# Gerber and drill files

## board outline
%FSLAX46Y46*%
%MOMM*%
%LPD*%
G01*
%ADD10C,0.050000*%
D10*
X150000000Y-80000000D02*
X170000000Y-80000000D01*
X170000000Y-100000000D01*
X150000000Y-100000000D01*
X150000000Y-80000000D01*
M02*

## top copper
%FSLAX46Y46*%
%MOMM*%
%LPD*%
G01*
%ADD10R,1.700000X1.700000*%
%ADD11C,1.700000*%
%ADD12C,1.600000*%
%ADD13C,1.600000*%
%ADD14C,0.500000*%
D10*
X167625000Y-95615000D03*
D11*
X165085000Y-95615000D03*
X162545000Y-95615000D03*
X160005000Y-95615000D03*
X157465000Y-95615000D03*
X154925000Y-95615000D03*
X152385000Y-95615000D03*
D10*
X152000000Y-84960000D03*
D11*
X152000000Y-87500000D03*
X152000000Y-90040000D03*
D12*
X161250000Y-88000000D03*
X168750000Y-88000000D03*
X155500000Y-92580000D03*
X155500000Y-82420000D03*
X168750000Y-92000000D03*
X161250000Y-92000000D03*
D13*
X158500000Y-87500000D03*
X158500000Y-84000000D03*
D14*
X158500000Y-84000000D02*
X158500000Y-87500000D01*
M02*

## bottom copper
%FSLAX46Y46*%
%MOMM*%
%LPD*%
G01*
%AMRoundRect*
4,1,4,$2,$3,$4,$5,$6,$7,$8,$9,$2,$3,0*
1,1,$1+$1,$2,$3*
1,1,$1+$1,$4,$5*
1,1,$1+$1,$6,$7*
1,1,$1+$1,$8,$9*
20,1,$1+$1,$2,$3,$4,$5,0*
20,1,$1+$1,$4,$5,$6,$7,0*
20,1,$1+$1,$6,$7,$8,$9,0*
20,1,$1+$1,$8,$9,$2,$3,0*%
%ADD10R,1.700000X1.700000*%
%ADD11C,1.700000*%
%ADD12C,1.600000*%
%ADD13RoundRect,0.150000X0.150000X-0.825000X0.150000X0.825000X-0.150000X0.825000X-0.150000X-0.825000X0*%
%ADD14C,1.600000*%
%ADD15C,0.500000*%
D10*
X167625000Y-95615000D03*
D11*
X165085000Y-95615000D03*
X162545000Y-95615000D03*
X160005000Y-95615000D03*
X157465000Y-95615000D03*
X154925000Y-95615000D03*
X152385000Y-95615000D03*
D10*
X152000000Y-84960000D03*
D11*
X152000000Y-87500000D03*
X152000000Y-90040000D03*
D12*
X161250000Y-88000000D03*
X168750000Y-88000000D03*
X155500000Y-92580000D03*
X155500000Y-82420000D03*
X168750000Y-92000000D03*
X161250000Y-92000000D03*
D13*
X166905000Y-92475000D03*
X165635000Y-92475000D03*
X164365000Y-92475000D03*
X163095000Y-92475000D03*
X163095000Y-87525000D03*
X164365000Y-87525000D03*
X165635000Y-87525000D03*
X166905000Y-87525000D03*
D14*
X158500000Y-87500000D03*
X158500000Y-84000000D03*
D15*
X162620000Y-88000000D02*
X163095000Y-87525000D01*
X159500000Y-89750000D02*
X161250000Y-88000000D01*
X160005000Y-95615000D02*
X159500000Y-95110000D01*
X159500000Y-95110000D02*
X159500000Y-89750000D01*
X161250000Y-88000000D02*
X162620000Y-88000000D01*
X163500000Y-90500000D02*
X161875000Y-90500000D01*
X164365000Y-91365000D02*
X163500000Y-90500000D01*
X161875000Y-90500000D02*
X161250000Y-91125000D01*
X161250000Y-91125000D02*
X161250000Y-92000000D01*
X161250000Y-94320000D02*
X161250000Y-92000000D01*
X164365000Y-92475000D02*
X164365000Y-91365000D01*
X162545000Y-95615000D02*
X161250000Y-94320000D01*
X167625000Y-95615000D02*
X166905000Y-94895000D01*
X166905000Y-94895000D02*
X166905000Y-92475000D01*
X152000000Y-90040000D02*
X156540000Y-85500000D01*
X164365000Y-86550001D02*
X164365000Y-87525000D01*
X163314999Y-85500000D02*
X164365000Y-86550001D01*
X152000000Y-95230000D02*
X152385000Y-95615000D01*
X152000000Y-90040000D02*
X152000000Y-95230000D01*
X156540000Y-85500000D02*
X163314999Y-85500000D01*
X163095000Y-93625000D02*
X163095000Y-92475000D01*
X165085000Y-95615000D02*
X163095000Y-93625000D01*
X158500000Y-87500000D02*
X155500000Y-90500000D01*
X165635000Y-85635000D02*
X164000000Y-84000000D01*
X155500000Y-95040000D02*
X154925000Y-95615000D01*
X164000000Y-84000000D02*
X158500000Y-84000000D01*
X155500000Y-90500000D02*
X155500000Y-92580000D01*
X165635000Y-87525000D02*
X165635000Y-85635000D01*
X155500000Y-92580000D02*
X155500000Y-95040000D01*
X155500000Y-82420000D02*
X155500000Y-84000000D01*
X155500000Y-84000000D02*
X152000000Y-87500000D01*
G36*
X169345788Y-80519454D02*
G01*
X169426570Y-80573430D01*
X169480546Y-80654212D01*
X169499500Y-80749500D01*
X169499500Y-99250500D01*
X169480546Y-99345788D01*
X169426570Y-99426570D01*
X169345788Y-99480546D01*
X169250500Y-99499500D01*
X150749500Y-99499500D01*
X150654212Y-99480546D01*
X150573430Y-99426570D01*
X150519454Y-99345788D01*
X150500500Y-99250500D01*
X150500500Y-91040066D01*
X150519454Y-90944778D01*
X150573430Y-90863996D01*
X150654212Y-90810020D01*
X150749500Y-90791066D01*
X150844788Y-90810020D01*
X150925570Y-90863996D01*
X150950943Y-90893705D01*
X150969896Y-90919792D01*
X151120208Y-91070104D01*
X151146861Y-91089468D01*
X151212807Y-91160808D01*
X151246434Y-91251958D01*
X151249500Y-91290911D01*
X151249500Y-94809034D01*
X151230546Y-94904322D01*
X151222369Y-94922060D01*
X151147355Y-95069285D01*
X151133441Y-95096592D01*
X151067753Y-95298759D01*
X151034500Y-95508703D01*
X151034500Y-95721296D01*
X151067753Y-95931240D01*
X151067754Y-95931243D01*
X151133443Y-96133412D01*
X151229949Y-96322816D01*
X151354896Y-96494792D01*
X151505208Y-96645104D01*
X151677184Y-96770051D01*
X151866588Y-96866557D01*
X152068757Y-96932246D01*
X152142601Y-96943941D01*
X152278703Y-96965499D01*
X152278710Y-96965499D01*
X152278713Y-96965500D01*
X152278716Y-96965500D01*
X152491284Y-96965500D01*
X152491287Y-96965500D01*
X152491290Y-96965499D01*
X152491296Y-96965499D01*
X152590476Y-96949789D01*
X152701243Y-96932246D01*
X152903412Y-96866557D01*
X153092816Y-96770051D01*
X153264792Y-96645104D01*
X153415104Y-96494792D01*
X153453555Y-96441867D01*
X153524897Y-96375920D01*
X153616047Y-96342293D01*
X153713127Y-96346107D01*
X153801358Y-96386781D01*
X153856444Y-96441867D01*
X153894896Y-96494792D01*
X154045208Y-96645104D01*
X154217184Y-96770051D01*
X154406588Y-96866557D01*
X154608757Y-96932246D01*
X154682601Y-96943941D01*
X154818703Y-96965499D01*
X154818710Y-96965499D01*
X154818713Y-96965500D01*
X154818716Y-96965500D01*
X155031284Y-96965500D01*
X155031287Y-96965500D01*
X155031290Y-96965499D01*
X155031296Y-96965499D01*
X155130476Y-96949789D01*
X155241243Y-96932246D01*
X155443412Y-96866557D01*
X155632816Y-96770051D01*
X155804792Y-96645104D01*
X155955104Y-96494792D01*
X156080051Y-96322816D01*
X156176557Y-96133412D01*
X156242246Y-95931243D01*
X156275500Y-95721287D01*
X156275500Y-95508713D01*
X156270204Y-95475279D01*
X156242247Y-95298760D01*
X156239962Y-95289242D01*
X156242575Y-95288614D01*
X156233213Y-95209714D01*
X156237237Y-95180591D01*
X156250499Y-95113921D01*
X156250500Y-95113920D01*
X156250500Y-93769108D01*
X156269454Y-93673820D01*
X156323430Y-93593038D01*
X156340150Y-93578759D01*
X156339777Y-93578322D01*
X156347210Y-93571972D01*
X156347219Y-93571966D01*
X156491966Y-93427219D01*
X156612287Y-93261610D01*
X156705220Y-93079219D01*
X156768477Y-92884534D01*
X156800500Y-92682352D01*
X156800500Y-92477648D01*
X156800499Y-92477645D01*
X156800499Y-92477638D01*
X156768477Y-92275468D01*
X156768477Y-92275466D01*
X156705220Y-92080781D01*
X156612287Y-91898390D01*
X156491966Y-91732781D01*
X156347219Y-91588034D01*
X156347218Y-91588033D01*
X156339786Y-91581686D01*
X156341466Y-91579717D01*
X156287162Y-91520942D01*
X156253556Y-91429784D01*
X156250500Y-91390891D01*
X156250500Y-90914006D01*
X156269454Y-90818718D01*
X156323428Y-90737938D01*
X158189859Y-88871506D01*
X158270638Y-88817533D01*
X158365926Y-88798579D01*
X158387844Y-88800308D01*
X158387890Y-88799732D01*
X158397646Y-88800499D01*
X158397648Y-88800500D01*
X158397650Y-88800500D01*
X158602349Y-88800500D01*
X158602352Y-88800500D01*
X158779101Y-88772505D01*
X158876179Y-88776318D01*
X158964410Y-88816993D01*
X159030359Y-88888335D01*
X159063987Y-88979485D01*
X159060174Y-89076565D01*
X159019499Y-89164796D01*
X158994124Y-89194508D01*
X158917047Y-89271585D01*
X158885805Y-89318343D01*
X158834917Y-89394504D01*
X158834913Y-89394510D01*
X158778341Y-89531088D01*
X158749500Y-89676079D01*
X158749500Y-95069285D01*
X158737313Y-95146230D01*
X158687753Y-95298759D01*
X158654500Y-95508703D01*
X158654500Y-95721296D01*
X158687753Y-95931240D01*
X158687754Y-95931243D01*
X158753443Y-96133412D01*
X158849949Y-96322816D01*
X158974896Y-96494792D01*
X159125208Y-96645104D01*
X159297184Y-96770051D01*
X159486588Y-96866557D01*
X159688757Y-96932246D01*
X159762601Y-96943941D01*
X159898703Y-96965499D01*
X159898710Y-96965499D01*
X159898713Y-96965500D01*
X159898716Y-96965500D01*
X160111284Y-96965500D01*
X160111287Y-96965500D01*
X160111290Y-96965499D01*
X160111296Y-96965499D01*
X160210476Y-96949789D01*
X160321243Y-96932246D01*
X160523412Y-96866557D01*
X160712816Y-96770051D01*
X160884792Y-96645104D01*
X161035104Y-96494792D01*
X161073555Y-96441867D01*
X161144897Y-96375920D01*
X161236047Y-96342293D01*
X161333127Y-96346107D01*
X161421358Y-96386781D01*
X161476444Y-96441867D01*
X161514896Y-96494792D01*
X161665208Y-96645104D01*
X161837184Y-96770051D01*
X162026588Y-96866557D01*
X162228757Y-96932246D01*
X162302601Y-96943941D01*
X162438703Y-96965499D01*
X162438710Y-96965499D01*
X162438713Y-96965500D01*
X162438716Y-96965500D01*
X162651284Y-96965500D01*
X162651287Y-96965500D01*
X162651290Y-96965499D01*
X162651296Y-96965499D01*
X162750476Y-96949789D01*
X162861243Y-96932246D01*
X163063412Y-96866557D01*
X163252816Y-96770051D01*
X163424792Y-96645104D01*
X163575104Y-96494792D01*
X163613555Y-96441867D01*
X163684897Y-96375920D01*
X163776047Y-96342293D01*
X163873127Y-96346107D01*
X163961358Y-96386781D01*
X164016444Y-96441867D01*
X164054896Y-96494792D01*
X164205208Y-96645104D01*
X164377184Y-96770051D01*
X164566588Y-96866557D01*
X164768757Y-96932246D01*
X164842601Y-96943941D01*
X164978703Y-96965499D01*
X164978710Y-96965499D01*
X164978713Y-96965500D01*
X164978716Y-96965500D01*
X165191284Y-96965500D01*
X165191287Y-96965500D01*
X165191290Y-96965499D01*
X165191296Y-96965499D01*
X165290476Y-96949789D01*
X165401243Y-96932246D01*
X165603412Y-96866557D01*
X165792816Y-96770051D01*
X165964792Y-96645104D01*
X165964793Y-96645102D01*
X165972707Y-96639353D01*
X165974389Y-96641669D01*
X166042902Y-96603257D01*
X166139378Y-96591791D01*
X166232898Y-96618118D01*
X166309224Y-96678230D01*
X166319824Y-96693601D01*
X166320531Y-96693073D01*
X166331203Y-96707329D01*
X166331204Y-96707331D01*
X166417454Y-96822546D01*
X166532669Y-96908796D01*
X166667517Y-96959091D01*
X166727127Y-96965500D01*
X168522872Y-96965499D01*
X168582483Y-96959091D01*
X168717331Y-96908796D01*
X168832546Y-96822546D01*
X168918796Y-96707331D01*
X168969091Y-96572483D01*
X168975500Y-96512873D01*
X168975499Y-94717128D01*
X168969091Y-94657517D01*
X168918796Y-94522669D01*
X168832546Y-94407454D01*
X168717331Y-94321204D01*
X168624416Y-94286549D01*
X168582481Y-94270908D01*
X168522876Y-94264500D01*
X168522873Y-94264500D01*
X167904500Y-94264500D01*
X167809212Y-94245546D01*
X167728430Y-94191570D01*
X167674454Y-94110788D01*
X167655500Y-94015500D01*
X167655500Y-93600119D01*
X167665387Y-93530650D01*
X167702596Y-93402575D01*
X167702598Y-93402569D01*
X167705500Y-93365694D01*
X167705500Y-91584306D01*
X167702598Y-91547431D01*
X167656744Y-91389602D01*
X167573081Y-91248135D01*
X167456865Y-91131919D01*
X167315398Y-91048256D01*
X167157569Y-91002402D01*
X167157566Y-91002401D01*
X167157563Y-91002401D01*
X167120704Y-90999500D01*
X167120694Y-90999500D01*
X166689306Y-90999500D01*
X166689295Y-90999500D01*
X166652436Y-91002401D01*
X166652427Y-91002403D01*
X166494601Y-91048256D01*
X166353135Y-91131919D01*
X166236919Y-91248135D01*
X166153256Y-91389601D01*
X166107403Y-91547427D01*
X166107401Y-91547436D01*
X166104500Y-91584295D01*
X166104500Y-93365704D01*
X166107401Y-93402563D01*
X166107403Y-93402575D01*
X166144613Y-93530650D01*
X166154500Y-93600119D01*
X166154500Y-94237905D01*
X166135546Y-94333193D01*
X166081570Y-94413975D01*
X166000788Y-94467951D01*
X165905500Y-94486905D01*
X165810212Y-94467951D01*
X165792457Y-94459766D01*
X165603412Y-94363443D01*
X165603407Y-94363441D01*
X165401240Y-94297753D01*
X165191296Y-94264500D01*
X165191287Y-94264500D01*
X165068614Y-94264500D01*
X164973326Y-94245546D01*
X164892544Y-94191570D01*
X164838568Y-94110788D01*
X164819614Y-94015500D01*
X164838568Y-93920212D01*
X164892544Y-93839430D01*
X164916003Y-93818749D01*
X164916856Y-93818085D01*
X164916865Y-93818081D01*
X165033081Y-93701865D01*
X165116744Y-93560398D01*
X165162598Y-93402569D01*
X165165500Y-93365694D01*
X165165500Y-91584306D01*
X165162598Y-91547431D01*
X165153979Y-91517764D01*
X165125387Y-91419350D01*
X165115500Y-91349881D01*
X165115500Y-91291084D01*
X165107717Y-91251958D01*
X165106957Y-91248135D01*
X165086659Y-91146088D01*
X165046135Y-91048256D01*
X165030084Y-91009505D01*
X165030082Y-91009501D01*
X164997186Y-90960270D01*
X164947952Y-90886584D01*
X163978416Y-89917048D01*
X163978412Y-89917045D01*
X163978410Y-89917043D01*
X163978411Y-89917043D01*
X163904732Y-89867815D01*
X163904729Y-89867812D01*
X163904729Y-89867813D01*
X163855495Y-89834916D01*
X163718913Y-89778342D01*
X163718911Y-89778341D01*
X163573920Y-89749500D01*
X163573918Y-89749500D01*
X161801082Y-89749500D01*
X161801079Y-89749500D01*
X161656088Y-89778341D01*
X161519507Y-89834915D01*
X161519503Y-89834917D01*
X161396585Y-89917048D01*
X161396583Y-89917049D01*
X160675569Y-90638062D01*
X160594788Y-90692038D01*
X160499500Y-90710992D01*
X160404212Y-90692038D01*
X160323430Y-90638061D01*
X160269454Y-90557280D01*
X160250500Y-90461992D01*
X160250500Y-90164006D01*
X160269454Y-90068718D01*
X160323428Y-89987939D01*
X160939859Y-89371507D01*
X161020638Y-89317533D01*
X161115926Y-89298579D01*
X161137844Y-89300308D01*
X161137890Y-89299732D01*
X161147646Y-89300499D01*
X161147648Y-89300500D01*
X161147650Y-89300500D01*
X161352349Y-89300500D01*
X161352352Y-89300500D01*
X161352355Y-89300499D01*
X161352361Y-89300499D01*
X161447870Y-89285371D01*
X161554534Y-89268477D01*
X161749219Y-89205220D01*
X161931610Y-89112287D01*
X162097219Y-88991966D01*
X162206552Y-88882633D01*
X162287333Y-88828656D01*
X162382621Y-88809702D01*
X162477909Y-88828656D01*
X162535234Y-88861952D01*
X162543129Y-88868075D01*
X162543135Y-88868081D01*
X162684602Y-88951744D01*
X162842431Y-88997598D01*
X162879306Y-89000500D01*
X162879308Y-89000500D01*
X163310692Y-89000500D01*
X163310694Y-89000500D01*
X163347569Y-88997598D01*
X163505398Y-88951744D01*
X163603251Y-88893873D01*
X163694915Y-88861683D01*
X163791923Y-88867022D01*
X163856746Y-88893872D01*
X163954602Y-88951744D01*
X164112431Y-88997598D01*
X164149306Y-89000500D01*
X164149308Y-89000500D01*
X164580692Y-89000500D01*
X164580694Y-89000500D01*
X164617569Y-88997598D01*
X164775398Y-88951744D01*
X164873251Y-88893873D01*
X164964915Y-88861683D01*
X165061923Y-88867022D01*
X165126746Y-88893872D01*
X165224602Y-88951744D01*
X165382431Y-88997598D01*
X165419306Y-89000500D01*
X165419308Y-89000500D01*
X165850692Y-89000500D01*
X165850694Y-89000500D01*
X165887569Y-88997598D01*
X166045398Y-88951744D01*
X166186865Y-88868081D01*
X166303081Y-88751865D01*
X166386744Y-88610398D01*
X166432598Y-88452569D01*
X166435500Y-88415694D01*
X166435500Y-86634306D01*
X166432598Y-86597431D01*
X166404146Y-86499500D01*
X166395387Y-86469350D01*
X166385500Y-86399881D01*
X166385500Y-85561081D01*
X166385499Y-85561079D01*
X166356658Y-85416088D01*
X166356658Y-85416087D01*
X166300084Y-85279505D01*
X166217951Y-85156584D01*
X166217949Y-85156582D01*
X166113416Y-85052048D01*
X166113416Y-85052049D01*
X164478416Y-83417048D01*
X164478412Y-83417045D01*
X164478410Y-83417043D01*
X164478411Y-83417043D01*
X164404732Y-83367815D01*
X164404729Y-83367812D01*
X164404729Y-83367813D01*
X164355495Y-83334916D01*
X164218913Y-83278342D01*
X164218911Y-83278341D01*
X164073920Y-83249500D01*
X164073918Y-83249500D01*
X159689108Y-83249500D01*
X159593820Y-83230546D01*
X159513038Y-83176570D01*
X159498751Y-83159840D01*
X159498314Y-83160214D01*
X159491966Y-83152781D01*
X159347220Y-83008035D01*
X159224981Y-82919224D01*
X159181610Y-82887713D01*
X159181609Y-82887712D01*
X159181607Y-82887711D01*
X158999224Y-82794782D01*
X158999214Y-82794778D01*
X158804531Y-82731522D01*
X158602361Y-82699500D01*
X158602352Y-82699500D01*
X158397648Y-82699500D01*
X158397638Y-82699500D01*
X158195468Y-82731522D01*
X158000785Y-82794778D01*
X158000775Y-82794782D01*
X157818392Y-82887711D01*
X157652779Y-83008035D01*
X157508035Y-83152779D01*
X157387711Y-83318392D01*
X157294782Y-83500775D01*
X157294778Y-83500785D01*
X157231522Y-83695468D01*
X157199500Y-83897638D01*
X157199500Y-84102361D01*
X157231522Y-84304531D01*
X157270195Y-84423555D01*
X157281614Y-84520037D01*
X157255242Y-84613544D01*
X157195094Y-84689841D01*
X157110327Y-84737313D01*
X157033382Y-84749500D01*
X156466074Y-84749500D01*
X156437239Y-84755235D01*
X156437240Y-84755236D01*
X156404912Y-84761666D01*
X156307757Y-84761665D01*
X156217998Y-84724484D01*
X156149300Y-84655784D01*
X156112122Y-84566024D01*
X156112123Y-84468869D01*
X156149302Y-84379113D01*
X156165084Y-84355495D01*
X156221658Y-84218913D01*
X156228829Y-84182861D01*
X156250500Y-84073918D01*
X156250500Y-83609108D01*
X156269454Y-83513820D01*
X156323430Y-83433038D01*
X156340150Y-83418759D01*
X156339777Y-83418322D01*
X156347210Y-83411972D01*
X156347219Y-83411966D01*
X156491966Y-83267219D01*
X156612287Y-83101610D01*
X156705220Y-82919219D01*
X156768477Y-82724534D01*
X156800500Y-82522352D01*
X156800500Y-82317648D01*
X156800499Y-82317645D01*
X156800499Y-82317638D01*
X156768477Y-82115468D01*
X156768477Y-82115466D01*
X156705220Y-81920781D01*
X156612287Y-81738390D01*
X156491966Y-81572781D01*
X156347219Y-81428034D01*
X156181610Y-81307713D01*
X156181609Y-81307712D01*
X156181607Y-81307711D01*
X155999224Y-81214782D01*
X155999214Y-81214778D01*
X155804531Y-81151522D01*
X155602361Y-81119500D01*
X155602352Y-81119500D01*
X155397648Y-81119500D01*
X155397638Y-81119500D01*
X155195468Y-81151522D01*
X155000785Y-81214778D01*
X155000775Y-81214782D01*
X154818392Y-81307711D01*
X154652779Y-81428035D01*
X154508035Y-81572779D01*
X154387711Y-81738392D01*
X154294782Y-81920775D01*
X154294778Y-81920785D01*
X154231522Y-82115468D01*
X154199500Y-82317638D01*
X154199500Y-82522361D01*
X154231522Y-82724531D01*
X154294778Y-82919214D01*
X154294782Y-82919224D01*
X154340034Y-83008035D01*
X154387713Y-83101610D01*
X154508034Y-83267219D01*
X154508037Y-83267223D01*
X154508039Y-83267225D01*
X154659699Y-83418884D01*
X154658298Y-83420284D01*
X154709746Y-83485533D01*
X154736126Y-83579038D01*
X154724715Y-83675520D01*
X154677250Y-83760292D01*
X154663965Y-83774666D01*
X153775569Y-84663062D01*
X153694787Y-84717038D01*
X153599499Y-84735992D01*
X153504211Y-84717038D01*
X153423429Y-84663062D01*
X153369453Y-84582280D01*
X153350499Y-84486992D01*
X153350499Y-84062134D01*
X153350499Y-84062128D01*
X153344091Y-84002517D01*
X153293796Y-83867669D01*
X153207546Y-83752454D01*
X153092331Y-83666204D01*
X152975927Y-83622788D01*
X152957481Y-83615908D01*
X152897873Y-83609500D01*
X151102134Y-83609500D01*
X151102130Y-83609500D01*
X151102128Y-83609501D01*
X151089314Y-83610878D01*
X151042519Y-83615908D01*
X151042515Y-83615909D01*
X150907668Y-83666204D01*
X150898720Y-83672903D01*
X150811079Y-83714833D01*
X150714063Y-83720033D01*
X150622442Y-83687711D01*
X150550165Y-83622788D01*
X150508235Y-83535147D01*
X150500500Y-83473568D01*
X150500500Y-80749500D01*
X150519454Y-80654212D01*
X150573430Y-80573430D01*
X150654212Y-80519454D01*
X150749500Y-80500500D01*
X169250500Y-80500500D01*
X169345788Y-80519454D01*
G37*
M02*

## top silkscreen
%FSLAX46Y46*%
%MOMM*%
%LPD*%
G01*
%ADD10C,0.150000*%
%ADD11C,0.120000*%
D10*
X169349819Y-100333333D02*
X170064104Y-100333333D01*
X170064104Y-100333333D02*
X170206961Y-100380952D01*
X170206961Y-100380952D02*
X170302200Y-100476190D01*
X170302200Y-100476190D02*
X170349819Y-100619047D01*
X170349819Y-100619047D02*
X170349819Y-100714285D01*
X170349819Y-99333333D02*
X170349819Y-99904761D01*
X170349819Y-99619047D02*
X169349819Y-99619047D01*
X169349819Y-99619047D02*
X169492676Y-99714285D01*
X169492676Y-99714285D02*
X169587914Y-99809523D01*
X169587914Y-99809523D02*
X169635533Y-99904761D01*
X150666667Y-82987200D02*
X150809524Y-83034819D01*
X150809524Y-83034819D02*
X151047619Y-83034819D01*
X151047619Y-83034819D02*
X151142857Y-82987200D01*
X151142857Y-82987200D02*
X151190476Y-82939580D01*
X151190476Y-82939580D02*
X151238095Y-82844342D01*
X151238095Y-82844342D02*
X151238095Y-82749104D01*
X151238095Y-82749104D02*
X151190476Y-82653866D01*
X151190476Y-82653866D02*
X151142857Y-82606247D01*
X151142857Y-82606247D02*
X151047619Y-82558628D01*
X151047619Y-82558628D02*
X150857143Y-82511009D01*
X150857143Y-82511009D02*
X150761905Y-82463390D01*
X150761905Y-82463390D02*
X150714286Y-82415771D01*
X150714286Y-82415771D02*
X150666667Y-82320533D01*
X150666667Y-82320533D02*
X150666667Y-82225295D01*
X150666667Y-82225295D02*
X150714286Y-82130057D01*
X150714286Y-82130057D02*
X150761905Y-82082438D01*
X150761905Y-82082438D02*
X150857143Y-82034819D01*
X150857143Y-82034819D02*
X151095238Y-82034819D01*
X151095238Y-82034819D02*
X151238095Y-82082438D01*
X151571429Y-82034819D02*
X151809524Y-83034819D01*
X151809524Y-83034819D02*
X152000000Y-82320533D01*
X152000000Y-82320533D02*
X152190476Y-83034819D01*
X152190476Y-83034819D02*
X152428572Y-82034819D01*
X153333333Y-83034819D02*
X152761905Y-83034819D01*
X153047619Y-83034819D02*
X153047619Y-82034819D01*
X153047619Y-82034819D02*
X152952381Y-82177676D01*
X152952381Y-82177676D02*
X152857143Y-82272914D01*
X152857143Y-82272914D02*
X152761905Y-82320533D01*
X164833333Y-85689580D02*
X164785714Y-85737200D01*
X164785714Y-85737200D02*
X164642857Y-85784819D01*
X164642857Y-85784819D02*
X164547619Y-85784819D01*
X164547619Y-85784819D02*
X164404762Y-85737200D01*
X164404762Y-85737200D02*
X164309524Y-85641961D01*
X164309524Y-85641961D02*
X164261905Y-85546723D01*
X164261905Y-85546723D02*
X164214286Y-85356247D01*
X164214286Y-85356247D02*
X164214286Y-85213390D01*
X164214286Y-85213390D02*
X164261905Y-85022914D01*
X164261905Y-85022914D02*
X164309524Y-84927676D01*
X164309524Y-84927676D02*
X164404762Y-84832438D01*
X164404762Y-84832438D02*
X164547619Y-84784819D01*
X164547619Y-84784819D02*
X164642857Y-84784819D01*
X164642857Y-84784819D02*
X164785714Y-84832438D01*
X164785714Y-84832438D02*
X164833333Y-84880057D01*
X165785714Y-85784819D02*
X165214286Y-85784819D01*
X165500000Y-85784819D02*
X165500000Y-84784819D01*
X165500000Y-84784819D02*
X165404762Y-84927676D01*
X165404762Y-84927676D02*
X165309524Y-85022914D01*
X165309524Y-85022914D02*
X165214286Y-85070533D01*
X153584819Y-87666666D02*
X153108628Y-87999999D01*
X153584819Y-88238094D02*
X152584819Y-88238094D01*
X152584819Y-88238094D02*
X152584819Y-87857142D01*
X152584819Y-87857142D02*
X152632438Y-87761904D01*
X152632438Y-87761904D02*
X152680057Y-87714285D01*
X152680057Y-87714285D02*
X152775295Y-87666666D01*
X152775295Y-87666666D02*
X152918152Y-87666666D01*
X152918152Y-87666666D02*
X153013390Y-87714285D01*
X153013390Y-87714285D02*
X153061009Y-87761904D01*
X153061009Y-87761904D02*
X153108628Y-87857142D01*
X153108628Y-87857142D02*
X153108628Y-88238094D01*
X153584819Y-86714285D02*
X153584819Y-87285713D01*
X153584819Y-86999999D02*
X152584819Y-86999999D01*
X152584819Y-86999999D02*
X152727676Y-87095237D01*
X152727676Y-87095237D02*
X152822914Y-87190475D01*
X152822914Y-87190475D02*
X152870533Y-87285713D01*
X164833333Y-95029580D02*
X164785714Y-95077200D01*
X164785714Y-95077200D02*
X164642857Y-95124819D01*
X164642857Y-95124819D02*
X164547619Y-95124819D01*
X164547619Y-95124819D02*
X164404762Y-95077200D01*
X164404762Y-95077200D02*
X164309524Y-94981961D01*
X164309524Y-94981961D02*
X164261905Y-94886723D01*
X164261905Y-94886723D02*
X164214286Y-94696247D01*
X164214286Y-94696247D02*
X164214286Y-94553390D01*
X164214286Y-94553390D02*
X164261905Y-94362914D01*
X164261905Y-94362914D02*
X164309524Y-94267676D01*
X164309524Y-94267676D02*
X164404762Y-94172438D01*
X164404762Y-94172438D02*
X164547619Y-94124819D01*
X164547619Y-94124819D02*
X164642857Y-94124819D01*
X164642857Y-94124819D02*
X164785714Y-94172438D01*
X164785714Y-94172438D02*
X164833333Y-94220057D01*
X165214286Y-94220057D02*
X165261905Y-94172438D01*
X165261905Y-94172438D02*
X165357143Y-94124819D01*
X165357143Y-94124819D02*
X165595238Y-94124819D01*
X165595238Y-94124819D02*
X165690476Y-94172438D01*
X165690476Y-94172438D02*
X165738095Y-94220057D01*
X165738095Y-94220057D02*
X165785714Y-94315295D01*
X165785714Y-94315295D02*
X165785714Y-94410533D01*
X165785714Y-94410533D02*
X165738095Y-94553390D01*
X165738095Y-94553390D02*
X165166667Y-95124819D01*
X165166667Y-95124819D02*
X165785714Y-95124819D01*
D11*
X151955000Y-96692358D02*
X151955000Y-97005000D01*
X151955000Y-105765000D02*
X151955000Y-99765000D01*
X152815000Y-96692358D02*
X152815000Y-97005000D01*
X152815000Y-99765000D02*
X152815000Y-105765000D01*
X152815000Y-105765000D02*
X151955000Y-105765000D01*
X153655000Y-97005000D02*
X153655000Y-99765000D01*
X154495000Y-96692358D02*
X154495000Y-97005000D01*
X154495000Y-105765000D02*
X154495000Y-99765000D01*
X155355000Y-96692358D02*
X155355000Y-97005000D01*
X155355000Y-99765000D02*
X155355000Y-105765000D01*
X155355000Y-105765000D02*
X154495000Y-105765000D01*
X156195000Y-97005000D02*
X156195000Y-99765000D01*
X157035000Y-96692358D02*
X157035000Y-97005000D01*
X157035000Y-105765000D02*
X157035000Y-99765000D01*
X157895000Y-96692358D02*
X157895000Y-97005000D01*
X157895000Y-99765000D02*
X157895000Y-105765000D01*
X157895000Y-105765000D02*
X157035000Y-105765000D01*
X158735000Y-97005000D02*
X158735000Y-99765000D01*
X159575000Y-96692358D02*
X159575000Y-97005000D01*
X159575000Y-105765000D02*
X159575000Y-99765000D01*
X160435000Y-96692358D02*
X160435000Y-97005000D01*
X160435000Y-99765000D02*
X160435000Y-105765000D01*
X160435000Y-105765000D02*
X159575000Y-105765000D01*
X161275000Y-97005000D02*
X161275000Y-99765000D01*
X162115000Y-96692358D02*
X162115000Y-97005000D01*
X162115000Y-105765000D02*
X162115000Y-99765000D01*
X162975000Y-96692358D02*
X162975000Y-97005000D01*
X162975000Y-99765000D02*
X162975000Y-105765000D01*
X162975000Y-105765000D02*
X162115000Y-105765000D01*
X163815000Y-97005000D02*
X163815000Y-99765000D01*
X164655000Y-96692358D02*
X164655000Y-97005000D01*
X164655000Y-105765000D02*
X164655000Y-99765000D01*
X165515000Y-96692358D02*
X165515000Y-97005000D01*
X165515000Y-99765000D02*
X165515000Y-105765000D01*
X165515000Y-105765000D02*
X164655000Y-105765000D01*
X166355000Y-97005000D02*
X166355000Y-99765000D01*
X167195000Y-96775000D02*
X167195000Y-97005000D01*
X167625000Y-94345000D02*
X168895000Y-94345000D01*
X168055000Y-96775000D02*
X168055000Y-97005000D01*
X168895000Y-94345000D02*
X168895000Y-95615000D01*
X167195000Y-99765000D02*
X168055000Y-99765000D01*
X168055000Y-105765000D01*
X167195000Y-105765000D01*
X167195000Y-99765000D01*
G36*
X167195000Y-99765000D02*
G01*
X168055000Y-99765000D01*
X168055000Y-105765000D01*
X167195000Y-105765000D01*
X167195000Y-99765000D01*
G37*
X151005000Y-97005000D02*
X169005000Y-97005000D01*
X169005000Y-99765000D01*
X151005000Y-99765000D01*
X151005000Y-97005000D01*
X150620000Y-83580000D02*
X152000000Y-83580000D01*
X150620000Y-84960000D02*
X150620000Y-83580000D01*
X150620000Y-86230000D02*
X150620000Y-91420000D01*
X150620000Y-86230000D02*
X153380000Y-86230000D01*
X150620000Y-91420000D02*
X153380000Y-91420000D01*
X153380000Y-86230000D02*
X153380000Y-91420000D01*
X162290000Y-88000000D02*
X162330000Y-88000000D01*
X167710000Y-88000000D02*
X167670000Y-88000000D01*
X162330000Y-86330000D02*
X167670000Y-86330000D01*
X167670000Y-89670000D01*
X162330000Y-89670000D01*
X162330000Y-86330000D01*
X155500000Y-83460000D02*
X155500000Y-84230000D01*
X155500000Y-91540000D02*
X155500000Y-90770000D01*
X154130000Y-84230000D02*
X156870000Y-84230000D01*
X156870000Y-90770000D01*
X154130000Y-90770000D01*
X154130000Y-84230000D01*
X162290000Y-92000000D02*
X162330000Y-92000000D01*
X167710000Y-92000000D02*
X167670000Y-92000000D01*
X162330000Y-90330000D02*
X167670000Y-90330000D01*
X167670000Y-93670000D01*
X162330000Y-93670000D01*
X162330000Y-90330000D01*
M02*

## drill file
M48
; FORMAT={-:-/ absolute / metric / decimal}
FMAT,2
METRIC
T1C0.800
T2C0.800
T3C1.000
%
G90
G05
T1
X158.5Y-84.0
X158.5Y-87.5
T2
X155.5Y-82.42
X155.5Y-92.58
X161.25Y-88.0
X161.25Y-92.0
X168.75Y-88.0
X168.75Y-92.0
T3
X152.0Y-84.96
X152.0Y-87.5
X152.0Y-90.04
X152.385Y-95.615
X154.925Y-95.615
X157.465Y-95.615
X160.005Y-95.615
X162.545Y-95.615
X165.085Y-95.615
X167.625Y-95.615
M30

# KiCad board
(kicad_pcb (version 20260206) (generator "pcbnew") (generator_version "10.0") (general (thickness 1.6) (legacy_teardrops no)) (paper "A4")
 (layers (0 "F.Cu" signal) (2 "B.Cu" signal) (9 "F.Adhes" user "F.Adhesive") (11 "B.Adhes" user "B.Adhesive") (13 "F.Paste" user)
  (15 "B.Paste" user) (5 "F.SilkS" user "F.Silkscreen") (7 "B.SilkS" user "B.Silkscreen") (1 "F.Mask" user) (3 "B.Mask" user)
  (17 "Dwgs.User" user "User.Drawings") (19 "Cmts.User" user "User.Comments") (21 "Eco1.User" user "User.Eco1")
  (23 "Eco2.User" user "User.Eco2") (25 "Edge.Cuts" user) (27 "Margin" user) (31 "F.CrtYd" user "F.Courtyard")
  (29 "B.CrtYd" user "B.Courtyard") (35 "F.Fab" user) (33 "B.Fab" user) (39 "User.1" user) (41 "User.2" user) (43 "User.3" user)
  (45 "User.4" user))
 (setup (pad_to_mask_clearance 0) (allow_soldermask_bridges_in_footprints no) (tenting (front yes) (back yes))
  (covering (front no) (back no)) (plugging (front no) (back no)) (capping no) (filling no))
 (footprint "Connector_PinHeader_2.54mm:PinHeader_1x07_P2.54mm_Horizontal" (layer "F.Cu") (at 167.625 95.615 -90)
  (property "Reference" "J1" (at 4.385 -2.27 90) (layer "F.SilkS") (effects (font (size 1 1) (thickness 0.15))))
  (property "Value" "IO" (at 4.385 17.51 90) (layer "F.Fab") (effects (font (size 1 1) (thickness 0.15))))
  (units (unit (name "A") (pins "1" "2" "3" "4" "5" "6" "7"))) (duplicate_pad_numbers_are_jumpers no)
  (fp_line (start 1.077358 15.67) (end 1.39 15.67) (stroke (width 0.12) (type solid)) (layer "F.SilkS"))
  (fp_line (start 10.15 15.67) (end 4.15 15.67) (stroke (width 0.12) (type solid)) (layer "F.SilkS"))
  (fp_line (start 1.077358 14.81) (end 1.39 14.81) (stroke (width 0.12) (type solid)) (layer "F.SilkS"))
  (fp_line (start 4.15 14.81) (end 10.15 14.81) (stroke (width 0.12) (type solid)) (layer "F.SilkS"))
  (fp_line (start 10.15 14.81) (end 10.15 15.67) (stroke (width 0.12) (type solid)) (layer "F.SilkS"))
  (fp_line (start 1.39 13.97) (end 4.15 13.97) (stroke (width 0.12) (type solid)) (layer "F.SilkS"))
  (fp_line (start 1.077358 13.13) (end 1.39 13.13) (stroke (width 0.12) (type solid)) (layer "F.SilkS"))
  (fp_line (start 10.15 13.13) (end 4.15 13.13) (stroke (width 0.12) (type solid)) (layer "F.SilkS"))
  (fp_line (start 1.077358 12.27) (end 1.39 12.27) (stroke (width 0.12) (type solid)) (layer "F.SilkS"))
  (fp_line (start 4.15 12.27) (end 10.15 12.27) (stroke (width 0.12) (type solid)) (layer "F.SilkS"))
  (fp_line (start 10.15 12.27) (end 10.15 13.13) (stroke (width 0.12) (type solid)) (layer "F.SilkS"))
  (fp_line (start 1.39 11.43) (end 4.15 11.43) (stroke (width 0.12) (type solid)) (layer "F.SilkS"))
  (fp_line (start 1.077358 10.59) (end 1.39 10.59) (stroke (width 0.12) (type solid)) (layer "F.SilkS"))
  (fp_line (start 10.15 10.59) (end 4.15 10.59) (stroke (width 0.12) (type solid)) (layer "F.SilkS"))
  (fp_line (start 1.077358 9.73) (end 1.39 9.73) (stroke (width 0.12) (type solid)) (layer "F.SilkS"))
  (fp_line (start 4.15 9.73) (end 10.15 9.73) (stroke (width 0.12) (type solid)) (layer "F.SilkS"))
  (fp_line (start 10.15 9.73) (end 10.15 10.59) (stroke (width 0.12) (type solid)) (layer "F.SilkS"))
  (fp_line (start 1.39 8.89) (end 4.15 8.89) (stroke (width 0.12) (type solid)) (layer "F.SilkS"))
  (fp_line (start 1.077358 8.05) (end 1.39 8.05) (stroke (width 0.12) (type solid)) (layer "F.SilkS"))
  (fp_line (start 10.15 8.05) (end 4.15 8.05) (stroke (width 0.12) (type solid)) (layer "F.SilkS"))
  (fp_line (start 1.077358 7.19) (end 1.39 7.19) (stroke (width 0.12) (type solid)) (layer "F.SilkS"))
  (fp_line (start 4.15 7.19) (end 10.15 7.19) (stroke (width 0.12) (type solid)) (layer "F.SilkS"))
  (fp_line (start 10.15 7.19) (end 10.15 8.05) (stroke (width 0.12) (type solid)) (layer "F.SilkS"))
  (fp_line (start 1.39 6.35) (end 4.15 6.35) (stroke (width 0.12) (type solid)) (layer "F.SilkS"))
  (fp_line (start 1.077358 5.51) (end 1.39 5.51) (stroke (width 0.12) (type solid)) (layer "F.SilkS"))
  (fp_line (start 10.15 5.51) (end 4.15 5.51) (stroke (width 0.12) (type solid)) (layer "F.SilkS"))
  (fp_line (start 1.077358 4.65) (end 1.39 4.65) (stroke (width 0.12) (type solid)) (layer "F.SilkS"))
  (fp_line (start 4.15 4.65) (end 10.15 4.65) (stroke (width 0.12) (type solid)) (layer "F.SilkS"))
  (fp_line (start 10.15 4.65) (end 10.15 5.51) (stroke (width 0.12) (type solid)) (layer "F.SilkS"))
  (fp_line (start 1.39 3.81) (end 4.15 3.81) (stroke (width 0.12) (type solid)) (layer "F.SilkS"))
  (fp_line (start 1.077358 2.97) (end 1.39 2.97) (stroke (width 0.12) (type solid)) (layer "F.SilkS"))
  (fp_line (start 10.15 2.97) (end 4.15 2.97) (stroke (width 0.12) (type solid)) (layer "F.SilkS"))
  (fp_line (start 1.077358 2.11) (end 1.39 2.11) (stroke (width 0.12) (type solid)) (layer "F.SilkS"))
  (fp_line (start 4.15 2.11) (end 10.15 2.11) (stroke (width 0.12) (type solid)) (layer "F.SilkS"))
  (fp_line (start 10.15 2.11) (end 10.15 2.97) (stroke (width 0.12) (type solid)) (layer "F.SilkS"))
  (fp_line (start 1.39 1.27) (end 4.15 1.27) (stroke (width 0.12) (type solid)) (layer "F.SilkS"))
  (fp_line (start 1.16 0.43) (end 1.39 0.43) (stroke (width 0.12) (type solid)) (layer "F.SilkS"))
  (fp_line (start -1.27 0) (end -1.27 -1.27) (stroke (width 0.12) (type solid)) (layer "F.SilkS"))
  (fp_line (start 1.16 -0.43) (end 1.39 -0.43) (stroke (width 0.12) (type solid)) (layer "F.SilkS"))
  (fp_line (start -1.27 -1.27) (end 0 -1.27) (stroke (width 0.12) (type solid)) (layer "F.SilkS"))
  (fp_rect (start 4.15 -0.43) (end 10.15 0.43) (stroke (width 0.12) (type solid)) (fill yes) (layer "F.SilkS"))
  (fp_rect (start 1.39 -1.38) (end 4.15 16.62) (stroke (width 0.12) (type solid)) (fill no) (layer "F.SilkS"))
  (pad "1" thru_hole rect (at 0 0 270) (size 1.7 1.7) (drill 1) (layers "*.Cu" "*.Mask") (remove_unused_layers no) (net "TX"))
  (pad "2" thru_hole circle (at 0 2.54 270) (size 1.7 1.7) (drill 1) (layers "*.Cu" "*.Mask") (remove_unused_layers no) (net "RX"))
  (pad "3" thru_hole circle (at 0 5.08 270) (size 1.7 1.7) (drill 1) (layers "*.Cu" "*.Mask") (remove_unused_layers no) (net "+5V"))
  (pad "4" thru_hole circle (at 0 7.62 270) (size 1.7 1.7) (drill 1) (layers "*.Cu" "*.Mask") (remove_unused_layers no) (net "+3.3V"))
  (pad "5" thru_hole circle (at 0 10.16 270) (size 1.7 1.7) (drill 1) (layers "*.Cu" "*.Mask") (remove_unused_layers no) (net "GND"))
  (pad "6" thru_hole circle (at 0 12.7 270) (size 1.7 1.7) (drill 1) (layers "*.Cu" "*.Mask") (remove_unused_layers no) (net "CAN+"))
  (pad "7" thru_hole circle (at 0 15.24 270) (size 1.7 1.7) (drill 1) (layers "*.Cu" "*.Mask") (remove_unused_layers no) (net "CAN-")))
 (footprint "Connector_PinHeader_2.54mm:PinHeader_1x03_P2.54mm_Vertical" (layer "F.Cu") (at 152 84.96)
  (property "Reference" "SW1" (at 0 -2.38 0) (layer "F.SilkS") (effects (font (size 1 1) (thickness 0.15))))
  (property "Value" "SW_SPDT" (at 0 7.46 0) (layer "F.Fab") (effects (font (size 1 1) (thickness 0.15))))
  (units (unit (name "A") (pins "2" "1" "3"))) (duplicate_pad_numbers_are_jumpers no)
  (fp_line (start -1.38 -1.38) (end 0 -1.38) (stroke (width 0.12) (type solid)) (layer "F.SilkS"))
  (fp_line (start -1.38 0) (end -1.38 -1.38) (stroke (width 0.12) (type solid)) (layer "F.SilkS"))
  (fp_line (start -1.38 1.27) (end -1.38 6.46) (stroke (width 0.12) (type solid)) (layer "F.SilkS"))
  (fp_line (start -1.38 1.27) (end 1.38 1.27) (stroke (width 0.12) (type solid)) (layer "F.SilkS"))
  (fp_line (start -1.38 6.46) (end 1.38 6.46) (stroke (width 0.12) (type solid)) (layer "F.SilkS"))
  (fp_line (start 1.38 1.27) (end 1.38 6.46) (stroke (width 0.12) (type solid)) (layer "F.SilkS"))
  (pad "1" thru_hole rect (at 0 0) (size 1.7 1.7) (drill 1) (layers "*.Cu" "*.Mask") (remove_unused_layers no)
   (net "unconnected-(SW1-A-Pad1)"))
  (pad "2" thru_hole circle (at 0 2.54) (size 1.7 1.7) (drill 1) (layers "*.Cu" "*.Mask") (remove_unused_layers no) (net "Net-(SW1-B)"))
  (pad "3" thru_hole circle (at 0 5.08) (size 1.7 1.7) (drill 1) (layers "*.Cu" "*.Mask") (remove_unused_layers no) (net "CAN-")))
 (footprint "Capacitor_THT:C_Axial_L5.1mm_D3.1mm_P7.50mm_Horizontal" (layer "F.Cu") (at 161.25 88)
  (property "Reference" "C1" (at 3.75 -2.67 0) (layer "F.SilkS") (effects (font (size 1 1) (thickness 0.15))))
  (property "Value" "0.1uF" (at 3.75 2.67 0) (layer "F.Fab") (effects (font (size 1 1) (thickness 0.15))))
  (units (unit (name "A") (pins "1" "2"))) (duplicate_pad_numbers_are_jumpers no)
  (fp_line (start 1.04 0) (end 1.08 0) (stroke (width 0.12) (type solid)) (layer "F.SilkS"))
  (fp_line (start 6.46 0) (end 6.42 0) (stroke (width 0.12) (type solid)) (layer "F.SilkS"))
  (fp_rect (start 1.08 -1.67) (end 6.42 1.67) (stroke (width 0.12) (type solid)) (fill no) (layer "F.SilkS"))
  (pad "1" thru_hole circle (at 0 0) (size 1.6 1.6) (drill 0.8) (layers "*.Cu" "*.Mask") (remove_unused_layers no) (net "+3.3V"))
  (pad "2" thru_hole circle (at 7.5 0) (size 1.6 1.6) (drill 0.8) (layers "*.Cu" "*.Mask") (remove_unused_layers no) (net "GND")))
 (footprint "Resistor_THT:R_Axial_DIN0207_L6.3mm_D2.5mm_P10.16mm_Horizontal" (layer "F.Cu") (at 155.5 92.58 90)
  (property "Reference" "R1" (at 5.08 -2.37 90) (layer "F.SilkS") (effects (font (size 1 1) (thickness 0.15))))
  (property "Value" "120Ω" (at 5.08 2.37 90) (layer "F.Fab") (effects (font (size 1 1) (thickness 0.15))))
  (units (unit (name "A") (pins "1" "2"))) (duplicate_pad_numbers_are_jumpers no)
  (fp_line (start 9.12 0) (end 8.35 0) (stroke (width 0.12) (type solid)) (layer "F.SilkS"))
  (fp_line (start 1.04 0) (end 1.81 0) (stroke (width 0.12) (type solid)) (layer "F.SilkS"))
  (fp_rect (start 1.81 -1.37) (end 8.35 1.37) (stroke (width 0.12) (type solid)) (fill no) (layer "F.SilkS"))
  (pad "1" thru_hole circle (at 0 0 90) (size 1.6 1.6) (drill 0.8) (layers "*.Cu" "*.Mask") (remove_unused_layers no) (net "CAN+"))
  (pad "2" thru_hole circle (at 10.16 0 90) (size 1.6 1.6) (drill 0.8) (layers "*.Cu" "*.Mask") (remove_unused_layers no)
   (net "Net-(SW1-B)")))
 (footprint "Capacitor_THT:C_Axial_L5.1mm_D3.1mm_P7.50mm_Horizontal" (layer "F.Cu") (at 168.75 92 180)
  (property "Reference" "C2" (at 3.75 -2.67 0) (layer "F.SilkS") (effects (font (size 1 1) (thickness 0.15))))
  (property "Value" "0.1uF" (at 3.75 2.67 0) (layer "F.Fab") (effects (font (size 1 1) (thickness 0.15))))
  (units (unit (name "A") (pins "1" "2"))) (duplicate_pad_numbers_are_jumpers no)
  (fp_line (start 6.46 0) (end 6.42 0) (stroke (width 0.12) (type solid)) (layer "F.SilkS"))
  (fp_line (start 1.04 0) (end 1.08 0) (stroke (width 0.12) (type solid)) (layer "F.SilkS"))
  (fp_rect (start 1.08 -1.67) (end 6.42 1.67) (stroke (width 0.12) (type solid)) (fill no) (layer "F.SilkS"))
  (pad "1" thru_hole circle (at 0 0 180) (size 1.6 1.6) (drill 0.8) (layers "*.Cu" "*.Mask") (remove_unused_layers no) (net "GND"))
  (pad "2" thru_hole circle (at 7.5 0 180) (size 1.6 1.6) (drill 0.8) (layers "*.Cu" "*.Mask") (remove_unused_layers no) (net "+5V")))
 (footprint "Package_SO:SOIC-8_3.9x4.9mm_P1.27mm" (layer "B.Cu") (at 165 90 90)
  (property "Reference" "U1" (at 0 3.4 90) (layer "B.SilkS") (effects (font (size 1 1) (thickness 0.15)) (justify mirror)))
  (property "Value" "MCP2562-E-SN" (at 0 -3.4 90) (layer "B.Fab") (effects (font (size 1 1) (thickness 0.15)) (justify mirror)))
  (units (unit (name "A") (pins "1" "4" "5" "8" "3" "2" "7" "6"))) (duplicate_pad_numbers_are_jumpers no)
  (pad "1" smd roundrect (at -2.475 1.905 90) (size 1.95 0.6) (layers "B.Cu" "B.Mask" "B.Paste") (roundrect_rratio 0.25) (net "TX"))
  (pad "2" smd roundrect (at -2.475 0.635 90) (size 1.95 0.6) (layers "B.Cu" "B.Mask" "B.Paste") (roundrect_rratio 0.25) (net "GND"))
  (pad "3" smd roundrect (at -2.475 -0.635 90) (size 1.95 0.6) (layers "B.Cu" "B.Mask" "B.Paste") (roundrect_rratio 0.25) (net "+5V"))
  (pad "4" smd roundrect (at -2.475 -1.905 90) (size 1.95 0.6) (layers "B.Cu" "B.Mask" "B.Paste") (roundrect_rratio 0.25) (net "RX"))
  (pad "5" smd roundrect (at 2.475 -1.905 90) (size 1.95 0.6) (layers "B.Cu" "B.Mask" "B.Paste") (roundrect_rratio 0.25) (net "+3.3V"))
  (pad "6" smd roundrect (at 2.475 -0.635 90) (size 1.95 0.6) (layers "B.Cu" "B.Mask" "B.Paste") (roundrect_rratio 0.25) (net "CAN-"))
  (pad "7" smd roundrect (at 2.475 0.635 90) (size 1.95 0.6) (layers "B.Cu" "B.Mask" "B.Paste") (roundrect_rratio 0.25) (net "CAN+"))
  (pad "8" smd roundrect (at 2.475 1.905 90) (size 1.95 0.6) (layers "B.Cu" "B.Mask" "B.Paste") (roundrect_rratio 0.25) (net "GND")))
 (gr_rect (start 150 80) (end 170 100) (stroke (width 0.05) (type default)) (fill no) (layer "Edge.Cuts"))
 (segment (start 162.62 88) (end 163.095 87.525) (width 0.5) (layer "B.Cu") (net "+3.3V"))
 (segment (start 159.5 89.75) (end 161.25 88) (width 0.5) (layer "B.Cu") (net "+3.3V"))
 (segment (start 160.005 95.615) (end 159.5 95.11) (width 0.5) (layer "B.Cu") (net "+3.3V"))
 (segment (start 159.5 95.11) (end 159.5 89.75) (width 0.5) (layer "B.Cu") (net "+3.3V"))
 (segment (start 161.25 88) (end 162.62 88) (width 0.5) (layer "B.Cu") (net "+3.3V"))
 (segment (start 163.5 90.5) (end 161.875 90.5) (width 0.5) (layer "B.Cu") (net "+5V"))
 (segment (start 164.365 91.365) (end 163.5 90.5) (width 0.5) (layer "B.Cu") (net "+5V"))
 (segment (start 161.875 90.5) (end 161.25 91.125) (width 0.5) (layer "B.Cu") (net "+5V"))
 (segment (start 161.25 91.125) (end 161.25 92) (width 0.5) (layer "B.Cu") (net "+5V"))
 (segment (start 161.25 94.32) (end 161.25 92) (width 0.5) (layer "B.Cu") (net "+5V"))
 (segment (start 164.365 92.475) (end 164.365 91.365) (width 0.5) (layer "B.Cu") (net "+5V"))
 (segment (start 162.545 95.615) (end 161.25 94.32) (width 0.5) (layer "B.Cu") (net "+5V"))
 (segment (start 167.625 95.615) (end 166.905 94.895) (width 0.5) (layer "B.Cu") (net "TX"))
 (segment (start 166.905 94.895) (end 166.905 92.475) (width 0.5) (layer "B.Cu") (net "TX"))
 (segment (start 152 90.04) (end 156.54 85.5) (width 0.5) (layer "B.Cu") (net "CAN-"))
 (segment (start 164.365 86.550001) (end 164.365 87.525) (width 0.5) (layer "B.Cu") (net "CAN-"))
 (segment (start 163.314999 85.5) (end 164.365 86.550001) (width 0.5) (layer "B.Cu") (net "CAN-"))
 (segment (start 152 95.23) (end 152.385 95.615) (width 0.5) (layer "B.Cu") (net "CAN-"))
 (segment (start 152 90.04) (end 152 95.23) (width 0.5) (layer "B.Cu") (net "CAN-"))
 (segment (start 156.54 85.5) (end 163.314999 85.5) (width 0.5) (layer "B.Cu") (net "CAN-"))
 (segment (start 163.095 93.625) (end 163.095 92.475) (width 0.5) (layer "B.Cu") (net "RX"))
 (segment (start 165.085 95.615) (end 163.095 93.625) (width 0.5) (layer "B.Cu") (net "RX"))
 (segment (start 158.5 84) (end 158.5 87.5) (width 0.5) (layer "F.Cu") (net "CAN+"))
 (via (at 158.5 87.5) (size 1.6) (drill 0.8) (layers "F.Cu" "B.Cu") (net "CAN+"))
 (via (at 158.5 84) (size 1.6) (drill 0.8) (layers "F.Cu" "B.Cu") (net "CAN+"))
 (segment (start 158.5 87.5) (end 155.5 90.5) (width 0.5) (layer "B.Cu") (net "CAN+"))
 (segment (start 165.635 85.635) (end 164 84) (width 0.5) (layer "B.Cu") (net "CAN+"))
 (segment (start 155.5 95.04) (end 154.925 95.615) (width 0.5) (layer "B.Cu") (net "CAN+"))
 (segment (start 164 84) (end 158.5 84) (width 0.5) (layer "B.Cu") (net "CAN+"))
 (segment (start 155.5 90.5) (end 155.5 92.58) (width 0.5) (layer "B.Cu") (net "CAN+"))
 (segment (start 165.635 87.525) (end 165.635 85.635) (width 0.5) (layer "B.Cu") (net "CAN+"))
 (segment (start 155.5 92.58) (end 155.5 95.04) (width 0.5) (layer "B.Cu") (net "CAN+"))
 (segment (start 155.5 82.42) (end 155.5 84) (width 0.5) (layer "B.Cu") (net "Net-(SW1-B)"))
 (segment (start 155.5 84) (end 152 87.5) (width 0.5) (layer "B.Cu") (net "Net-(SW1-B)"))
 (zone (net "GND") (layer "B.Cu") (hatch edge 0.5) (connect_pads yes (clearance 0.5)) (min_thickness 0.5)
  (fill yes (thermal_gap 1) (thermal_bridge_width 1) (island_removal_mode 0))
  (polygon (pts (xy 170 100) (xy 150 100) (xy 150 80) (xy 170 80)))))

